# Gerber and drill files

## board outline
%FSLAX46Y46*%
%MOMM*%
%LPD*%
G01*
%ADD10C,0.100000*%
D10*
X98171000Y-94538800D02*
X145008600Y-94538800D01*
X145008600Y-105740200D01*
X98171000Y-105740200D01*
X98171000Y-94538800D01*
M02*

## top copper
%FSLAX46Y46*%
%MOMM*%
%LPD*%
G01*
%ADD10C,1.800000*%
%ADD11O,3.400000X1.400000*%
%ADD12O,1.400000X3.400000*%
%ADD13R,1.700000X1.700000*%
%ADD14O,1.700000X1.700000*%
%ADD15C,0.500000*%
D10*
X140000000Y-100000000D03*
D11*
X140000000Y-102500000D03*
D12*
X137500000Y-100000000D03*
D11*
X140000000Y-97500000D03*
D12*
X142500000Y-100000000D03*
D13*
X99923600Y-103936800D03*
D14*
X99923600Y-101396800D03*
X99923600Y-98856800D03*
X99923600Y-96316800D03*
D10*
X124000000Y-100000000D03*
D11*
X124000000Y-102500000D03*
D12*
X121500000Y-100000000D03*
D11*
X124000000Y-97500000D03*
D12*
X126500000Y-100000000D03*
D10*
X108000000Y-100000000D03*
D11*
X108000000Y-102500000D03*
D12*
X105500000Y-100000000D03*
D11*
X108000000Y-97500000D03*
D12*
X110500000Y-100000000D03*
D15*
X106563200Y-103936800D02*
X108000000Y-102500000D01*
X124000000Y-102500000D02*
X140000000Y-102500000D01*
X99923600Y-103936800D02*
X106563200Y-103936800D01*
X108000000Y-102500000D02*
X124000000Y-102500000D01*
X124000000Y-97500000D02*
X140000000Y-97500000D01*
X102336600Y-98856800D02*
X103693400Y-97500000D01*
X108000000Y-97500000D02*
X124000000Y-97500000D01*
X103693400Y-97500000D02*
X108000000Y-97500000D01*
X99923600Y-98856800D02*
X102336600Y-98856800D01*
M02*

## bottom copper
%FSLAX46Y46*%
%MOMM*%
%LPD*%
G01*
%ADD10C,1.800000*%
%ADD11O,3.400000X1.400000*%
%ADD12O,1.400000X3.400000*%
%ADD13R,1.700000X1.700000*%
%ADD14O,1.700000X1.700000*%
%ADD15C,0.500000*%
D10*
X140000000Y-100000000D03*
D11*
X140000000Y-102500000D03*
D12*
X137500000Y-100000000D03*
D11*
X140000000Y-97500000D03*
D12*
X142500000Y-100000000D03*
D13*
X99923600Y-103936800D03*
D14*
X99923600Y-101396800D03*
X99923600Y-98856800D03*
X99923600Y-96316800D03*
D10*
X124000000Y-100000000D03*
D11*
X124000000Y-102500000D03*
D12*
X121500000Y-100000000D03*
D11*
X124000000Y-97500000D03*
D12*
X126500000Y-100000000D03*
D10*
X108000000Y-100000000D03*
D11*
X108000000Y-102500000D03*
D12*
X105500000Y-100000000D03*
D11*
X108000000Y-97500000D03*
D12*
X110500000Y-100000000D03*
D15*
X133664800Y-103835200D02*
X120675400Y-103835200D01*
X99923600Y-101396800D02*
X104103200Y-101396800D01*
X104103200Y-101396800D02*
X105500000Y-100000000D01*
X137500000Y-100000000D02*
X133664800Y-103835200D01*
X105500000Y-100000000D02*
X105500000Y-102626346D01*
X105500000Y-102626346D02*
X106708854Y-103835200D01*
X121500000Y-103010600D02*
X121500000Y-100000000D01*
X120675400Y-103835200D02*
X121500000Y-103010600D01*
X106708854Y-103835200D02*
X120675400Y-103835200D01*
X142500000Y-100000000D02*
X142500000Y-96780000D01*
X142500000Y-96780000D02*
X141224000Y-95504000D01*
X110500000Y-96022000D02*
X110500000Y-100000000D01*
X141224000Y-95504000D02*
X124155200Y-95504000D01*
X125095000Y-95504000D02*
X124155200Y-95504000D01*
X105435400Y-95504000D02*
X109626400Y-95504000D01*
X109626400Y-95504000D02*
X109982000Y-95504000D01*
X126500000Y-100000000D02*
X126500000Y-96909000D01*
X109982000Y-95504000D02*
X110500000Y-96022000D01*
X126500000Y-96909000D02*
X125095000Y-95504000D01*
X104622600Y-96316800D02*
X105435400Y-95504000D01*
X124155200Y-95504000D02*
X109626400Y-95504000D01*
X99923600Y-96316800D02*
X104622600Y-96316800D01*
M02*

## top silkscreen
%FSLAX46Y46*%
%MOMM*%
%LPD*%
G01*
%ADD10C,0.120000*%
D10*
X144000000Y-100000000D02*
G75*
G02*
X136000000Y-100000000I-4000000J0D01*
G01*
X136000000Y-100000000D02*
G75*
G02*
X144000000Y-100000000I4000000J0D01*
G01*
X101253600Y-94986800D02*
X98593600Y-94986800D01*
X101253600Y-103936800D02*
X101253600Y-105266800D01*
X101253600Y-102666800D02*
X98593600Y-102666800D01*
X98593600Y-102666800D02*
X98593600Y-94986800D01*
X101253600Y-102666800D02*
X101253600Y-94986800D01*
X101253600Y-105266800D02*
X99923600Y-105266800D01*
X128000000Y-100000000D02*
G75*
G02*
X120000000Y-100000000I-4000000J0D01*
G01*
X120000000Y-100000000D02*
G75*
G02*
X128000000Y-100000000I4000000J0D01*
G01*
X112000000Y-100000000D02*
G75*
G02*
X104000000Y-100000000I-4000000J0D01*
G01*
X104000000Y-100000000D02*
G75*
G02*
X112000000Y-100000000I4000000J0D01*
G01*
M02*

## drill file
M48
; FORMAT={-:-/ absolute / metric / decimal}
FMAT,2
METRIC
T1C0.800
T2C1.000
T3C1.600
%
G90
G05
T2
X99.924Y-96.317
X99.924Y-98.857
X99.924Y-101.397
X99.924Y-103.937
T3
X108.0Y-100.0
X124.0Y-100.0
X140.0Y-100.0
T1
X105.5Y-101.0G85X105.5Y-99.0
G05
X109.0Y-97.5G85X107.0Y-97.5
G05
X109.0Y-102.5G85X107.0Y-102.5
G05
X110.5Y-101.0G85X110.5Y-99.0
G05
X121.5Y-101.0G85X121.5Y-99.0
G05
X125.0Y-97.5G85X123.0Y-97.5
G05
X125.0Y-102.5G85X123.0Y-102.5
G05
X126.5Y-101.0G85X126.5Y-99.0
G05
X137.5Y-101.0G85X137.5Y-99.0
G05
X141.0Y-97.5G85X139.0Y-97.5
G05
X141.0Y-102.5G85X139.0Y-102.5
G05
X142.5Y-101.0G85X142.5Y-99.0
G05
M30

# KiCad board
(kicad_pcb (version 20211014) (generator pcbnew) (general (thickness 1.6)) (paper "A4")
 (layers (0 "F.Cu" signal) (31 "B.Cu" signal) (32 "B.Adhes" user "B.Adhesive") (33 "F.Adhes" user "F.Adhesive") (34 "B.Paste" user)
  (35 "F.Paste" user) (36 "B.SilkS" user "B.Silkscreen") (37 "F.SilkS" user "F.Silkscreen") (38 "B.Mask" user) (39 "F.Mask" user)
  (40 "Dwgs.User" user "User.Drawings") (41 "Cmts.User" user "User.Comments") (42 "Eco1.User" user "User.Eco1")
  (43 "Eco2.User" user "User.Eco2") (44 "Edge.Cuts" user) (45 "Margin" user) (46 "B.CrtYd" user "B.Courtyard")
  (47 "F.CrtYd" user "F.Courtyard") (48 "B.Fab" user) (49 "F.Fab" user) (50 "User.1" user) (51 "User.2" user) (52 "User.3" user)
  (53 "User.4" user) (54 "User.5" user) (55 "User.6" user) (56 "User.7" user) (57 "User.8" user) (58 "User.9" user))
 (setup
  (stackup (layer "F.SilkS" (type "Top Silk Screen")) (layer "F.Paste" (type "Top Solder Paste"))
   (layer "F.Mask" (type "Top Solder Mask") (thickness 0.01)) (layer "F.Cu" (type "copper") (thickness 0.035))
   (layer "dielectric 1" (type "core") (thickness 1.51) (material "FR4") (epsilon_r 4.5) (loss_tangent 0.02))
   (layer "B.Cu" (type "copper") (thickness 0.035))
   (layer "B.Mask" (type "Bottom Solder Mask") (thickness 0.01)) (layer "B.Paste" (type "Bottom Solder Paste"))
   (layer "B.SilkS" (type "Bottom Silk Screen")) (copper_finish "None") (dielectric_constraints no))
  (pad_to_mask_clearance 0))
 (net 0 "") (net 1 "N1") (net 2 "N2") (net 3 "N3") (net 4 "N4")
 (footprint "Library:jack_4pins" (layer "F.Cu") (at 140 100)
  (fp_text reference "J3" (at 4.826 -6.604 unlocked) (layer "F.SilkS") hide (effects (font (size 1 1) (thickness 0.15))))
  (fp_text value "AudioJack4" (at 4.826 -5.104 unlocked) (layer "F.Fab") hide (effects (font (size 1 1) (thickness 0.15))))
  (fp_circle (center 0 0) (end 4 0) (layer "F.SilkS") (width 0.12) (fill none))
  (pad "" thru_hole circle (at 0 0) (size 1.8 1.8) (drill 1.6) (layers *.Mask))
  (pad "1" thru_hole oval (at 0 2.5 180) (size 3.4 1.4) (drill oval 2.8 0.8) (layers *.Cu *.Mask) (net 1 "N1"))
  (pad "2" thru_hole oval (at -2.5 0 90) (size 3.4 1.4) (drill oval 2.8 0.8) (layers *.Cu *.Mask) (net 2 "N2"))
  (pad "3" thru_hole oval (at 0 -2.5 180) (size 3.4 1.4) (drill oval 2.8 0.8) (layers *.Cu *.Mask) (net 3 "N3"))
  (pad "4" thru_hole oval (at 2.5 0 90) (size 3.4 1.4) (drill oval 2.8 0.8) (layers *.Cu *.Mask) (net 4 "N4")))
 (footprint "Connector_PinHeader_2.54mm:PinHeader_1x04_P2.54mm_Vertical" (layer "F.Cu") (at 99.9236 103.9368 180)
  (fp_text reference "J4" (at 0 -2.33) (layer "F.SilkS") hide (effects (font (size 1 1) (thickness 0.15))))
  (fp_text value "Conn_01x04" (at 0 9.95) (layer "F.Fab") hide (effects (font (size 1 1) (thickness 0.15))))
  (fp_line (start -1.33 8.95) (end 1.33 8.95) (layer "F.SilkS") (width 0.12))
  (fp_line (start -1.33 0) (end -1.33 -1.33) (layer "F.SilkS") (width 0.12))
  (fp_line (start -1.33 1.27) (end 1.33 1.27) (layer "F.SilkS") (width 0.12))
  (fp_line (start 1.33 1.27) (end 1.33 8.95) (layer "F.SilkS") (width 0.12))
  (fp_line (start -1.33 1.27) (end -1.33 8.95) (layer "F.SilkS") (width 0.12))
  (fp_line (start -1.33 -1.33) (end 0 -1.33) (layer "F.SilkS") (width 0.12))
  (pad "1" thru_hole rect (at 0 0 180) (size 1.7 1.7) (drill 1) (layers *.Cu *.Mask) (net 1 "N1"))
  (pad "2" thru_hole oval (at 0 2.54 180) (size 1.7 1.7) (drill 1) (layers *.Cu *.Mask) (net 2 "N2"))
  (pad "3" thru_hole oval (at 0 5.08 180) (size 1.7 1.7) (drill 1) (layers *.Cu *.Mask) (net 3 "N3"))
  (pad "4" thru_hole oval (at 0 7.62 180) (size 1.7 1.7) (drill 1) (layers *.Cu *.Mask) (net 4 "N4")))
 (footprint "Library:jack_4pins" (layer "F.Cu") (at 124 100)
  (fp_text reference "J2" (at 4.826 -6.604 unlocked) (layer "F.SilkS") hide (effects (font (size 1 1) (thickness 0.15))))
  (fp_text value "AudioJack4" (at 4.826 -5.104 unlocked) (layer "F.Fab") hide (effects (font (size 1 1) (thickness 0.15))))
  (fp_circle (center 0 0) (end 4 0) (layer "F.SilkS") (width 0.12) (fill none))
  (pad "" thru_hole circle (at 0 0) (size 1.8 1.8) (drill 1.6) (layers *.Mask))
  (pad "1" thru_hole oval (at 0 2.5 180) (size 3.4 1.4) (drill oval 2.8 0.8) (layers *.Cu *.Mask) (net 1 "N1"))
  (pad "2" thru_hole oval (at -2.5 0 90) (size 3.4 1.4) (drill oval 2.8 0.8) (layers *.Cu *.Mask) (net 2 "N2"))
  (pad "3" thru_hole oval (at 0 -2.5 180) (size 3.4 1.4) (drill oval 2.8 0.8) (layers *.Cu *.Mask) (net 3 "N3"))
  (pad "4" thru_hole oval (at 2.5 0 90) (size 3.4 1.4) (drill oval 2.8 0.8) (layers *.Cu *.Mask) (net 4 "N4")))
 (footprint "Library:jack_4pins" (layer "F.Cu") (at 108 100)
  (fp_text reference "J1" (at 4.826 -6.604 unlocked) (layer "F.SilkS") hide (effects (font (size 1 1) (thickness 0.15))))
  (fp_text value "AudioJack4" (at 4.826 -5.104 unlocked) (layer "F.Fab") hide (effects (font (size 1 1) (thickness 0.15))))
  (fp_circle (center 0 0) (end 4 0) (layer "F.SilkS") (width 0.12) (fill none))
  (pad "" thru_hole circle (at 0 0) (size 1.8 1.8) (drill 1.6) (layers *.Mask))
  (pad "1" thru_hole oval (at 0 2.5 180) (size 3.4 1.4) (drill oval 2.8 0.8) (layers *.Cu *.Mask) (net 1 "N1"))
  (pad "2" thru_hole oval (at -2.5 0 90) (size 3.4 1.4) (drill oval 2.8 0.8) (layers *.Cu *.Mask) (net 2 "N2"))
  (pad "3" thru_hole oval (at 0 -2.5 180) (size 3.4 1.4) (drill oval 2.8 0.8) (layers *.Cu *.Mask) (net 3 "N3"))
  (pad "4" thru_hole oval (at 2.5 0 90) (size 3.4 1.4) (drill oval 2.8 0.8) (layers *.Cu *.Mask) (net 4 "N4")))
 (gr_rect (start 98.171 94.5388) (end 145.0086 105.7402) (layer "Edge.Cuts") (width 0.1) (fill none))
 (segment (start 133.6648 103.8352) (end 120.6754 103.8352) (width 0.5) (layer "B.Cu") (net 2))
 (segment (start 99.9236 101.3968) (end 104.1032 101.3968) (width 0.5) (layer "B.Cu") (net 2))
 (segment (start 104.1032 101.3968) (end 105.5 100) (width 0.5) (layer "B.Cu") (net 2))
 (segment (start 137.5 100) (end 133.6648 103.8352) (width 0.5) (layer "B.Cu") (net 2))
 (segment (start 105.5 100) (end 105.5 102.626346) (width 0.5) (layer "B.Cu") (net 2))
 (segment (start 105.5 102.626346) (end 106.708854 103.8352) (width 0.5) (layer "B.Cu") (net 2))
 (segment (start 121.5 103.0106) (end 121.5 100) (width 0.5) (layer "B.Cu") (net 2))
 (segment (start 120.6754 103.8352) (end 121.5 103.0106) (width 0.5) (layer "B.Cu") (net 2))
 (segment (start 106.708854 103.8352) (end 120.6754 103.8352) (width 0.5) (layer "B.Cu") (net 2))
 (segment (start 106.5632 103.9368) (end 108 102.5) (width 0.5) (layer "F.Cu") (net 1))
 (segment (start 124 102.5) (end 140 102.5) (width 0.5) (layer "F.Cu") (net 1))
 (segment (start 99.9236 103.9368) (end 106.5632 103.9368) (width 0.5) (layer "F.Cu") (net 1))
 (segment (start 108 102.5) (end 124 102.5) (width 0.5) (layer "F.Cu") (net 1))
 (segment (start 142.5 100) (end 142.5 96.78) (width 0.5) (layer "B.Cu") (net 4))
 (segment (start 142.5 96.78) (end 141.224 95.504) (width 0.5) (layer "B.Cu") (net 4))
 (segment (start 110.5 96.022) (end 110.5 100) (width 0.5) (layer "B.Cu") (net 4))
 (segment (start 141.224 95.504) (end 124.1552 95.504) (width 0.5) (layer "B.Cu") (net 4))
 (segment (start 125.095 95.504) (end 124.1552 95.504) (width 0.5) (layer "B.Cu") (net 4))
 (segment (start 105.4354 95.504) (end 109.6264 95.504) (width 0.5) (layer "B.Cu") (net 4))
 (segment (start 109.6264 95.504) (end 109.982 95.504) (width 0.5) (layer "B.Cu") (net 4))
 (segment (start 126.5 100) (end 126.5 96.909) (width 0.5) (layer "B.Cu") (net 4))
 (segment (start 109.982 95.504) (end 110.5 96.022) (width 0.5) (layer "B.Cu") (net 4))
 (segment (start 126.5 96.909) (end 125.095 95.504) (width 0.5) (layer "B.Cu") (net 4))
 (segment (start 104.6226 96.3168) (end 105.4354 95.504) (width 0.5) (layer "B.Cu") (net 4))
 (segment (start 124.1552 95.504) (end 109.6264 95.504) (width 0.5) (layer "B.Cu") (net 4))
 (segment (start 99.9236 96.3168) (end 104.6226 96.3168) (width 0.5) (layer "B.Cu") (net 4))
 (segment (start 124 97.5) (end 140 97.5) (width 0.5) (layer "F.Cu") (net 3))
 (segment (start 102.3366 98.8568) (end 103.6934 97.5) (width 0.5) (layer "F.Cu") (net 3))
 (segment (start 108 97.5) (end 124 97.5) (width 0.5) (layer "F.Cu") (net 3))
 (segment (start 103.6934 97.5) (end 108 97.5) (width 0.5) (layer "F.Cu") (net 3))
 (segment (start 99.9236 98.8568) (end 102.3366 98.8568) (width 0.5) (layer "F.Cu") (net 3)))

